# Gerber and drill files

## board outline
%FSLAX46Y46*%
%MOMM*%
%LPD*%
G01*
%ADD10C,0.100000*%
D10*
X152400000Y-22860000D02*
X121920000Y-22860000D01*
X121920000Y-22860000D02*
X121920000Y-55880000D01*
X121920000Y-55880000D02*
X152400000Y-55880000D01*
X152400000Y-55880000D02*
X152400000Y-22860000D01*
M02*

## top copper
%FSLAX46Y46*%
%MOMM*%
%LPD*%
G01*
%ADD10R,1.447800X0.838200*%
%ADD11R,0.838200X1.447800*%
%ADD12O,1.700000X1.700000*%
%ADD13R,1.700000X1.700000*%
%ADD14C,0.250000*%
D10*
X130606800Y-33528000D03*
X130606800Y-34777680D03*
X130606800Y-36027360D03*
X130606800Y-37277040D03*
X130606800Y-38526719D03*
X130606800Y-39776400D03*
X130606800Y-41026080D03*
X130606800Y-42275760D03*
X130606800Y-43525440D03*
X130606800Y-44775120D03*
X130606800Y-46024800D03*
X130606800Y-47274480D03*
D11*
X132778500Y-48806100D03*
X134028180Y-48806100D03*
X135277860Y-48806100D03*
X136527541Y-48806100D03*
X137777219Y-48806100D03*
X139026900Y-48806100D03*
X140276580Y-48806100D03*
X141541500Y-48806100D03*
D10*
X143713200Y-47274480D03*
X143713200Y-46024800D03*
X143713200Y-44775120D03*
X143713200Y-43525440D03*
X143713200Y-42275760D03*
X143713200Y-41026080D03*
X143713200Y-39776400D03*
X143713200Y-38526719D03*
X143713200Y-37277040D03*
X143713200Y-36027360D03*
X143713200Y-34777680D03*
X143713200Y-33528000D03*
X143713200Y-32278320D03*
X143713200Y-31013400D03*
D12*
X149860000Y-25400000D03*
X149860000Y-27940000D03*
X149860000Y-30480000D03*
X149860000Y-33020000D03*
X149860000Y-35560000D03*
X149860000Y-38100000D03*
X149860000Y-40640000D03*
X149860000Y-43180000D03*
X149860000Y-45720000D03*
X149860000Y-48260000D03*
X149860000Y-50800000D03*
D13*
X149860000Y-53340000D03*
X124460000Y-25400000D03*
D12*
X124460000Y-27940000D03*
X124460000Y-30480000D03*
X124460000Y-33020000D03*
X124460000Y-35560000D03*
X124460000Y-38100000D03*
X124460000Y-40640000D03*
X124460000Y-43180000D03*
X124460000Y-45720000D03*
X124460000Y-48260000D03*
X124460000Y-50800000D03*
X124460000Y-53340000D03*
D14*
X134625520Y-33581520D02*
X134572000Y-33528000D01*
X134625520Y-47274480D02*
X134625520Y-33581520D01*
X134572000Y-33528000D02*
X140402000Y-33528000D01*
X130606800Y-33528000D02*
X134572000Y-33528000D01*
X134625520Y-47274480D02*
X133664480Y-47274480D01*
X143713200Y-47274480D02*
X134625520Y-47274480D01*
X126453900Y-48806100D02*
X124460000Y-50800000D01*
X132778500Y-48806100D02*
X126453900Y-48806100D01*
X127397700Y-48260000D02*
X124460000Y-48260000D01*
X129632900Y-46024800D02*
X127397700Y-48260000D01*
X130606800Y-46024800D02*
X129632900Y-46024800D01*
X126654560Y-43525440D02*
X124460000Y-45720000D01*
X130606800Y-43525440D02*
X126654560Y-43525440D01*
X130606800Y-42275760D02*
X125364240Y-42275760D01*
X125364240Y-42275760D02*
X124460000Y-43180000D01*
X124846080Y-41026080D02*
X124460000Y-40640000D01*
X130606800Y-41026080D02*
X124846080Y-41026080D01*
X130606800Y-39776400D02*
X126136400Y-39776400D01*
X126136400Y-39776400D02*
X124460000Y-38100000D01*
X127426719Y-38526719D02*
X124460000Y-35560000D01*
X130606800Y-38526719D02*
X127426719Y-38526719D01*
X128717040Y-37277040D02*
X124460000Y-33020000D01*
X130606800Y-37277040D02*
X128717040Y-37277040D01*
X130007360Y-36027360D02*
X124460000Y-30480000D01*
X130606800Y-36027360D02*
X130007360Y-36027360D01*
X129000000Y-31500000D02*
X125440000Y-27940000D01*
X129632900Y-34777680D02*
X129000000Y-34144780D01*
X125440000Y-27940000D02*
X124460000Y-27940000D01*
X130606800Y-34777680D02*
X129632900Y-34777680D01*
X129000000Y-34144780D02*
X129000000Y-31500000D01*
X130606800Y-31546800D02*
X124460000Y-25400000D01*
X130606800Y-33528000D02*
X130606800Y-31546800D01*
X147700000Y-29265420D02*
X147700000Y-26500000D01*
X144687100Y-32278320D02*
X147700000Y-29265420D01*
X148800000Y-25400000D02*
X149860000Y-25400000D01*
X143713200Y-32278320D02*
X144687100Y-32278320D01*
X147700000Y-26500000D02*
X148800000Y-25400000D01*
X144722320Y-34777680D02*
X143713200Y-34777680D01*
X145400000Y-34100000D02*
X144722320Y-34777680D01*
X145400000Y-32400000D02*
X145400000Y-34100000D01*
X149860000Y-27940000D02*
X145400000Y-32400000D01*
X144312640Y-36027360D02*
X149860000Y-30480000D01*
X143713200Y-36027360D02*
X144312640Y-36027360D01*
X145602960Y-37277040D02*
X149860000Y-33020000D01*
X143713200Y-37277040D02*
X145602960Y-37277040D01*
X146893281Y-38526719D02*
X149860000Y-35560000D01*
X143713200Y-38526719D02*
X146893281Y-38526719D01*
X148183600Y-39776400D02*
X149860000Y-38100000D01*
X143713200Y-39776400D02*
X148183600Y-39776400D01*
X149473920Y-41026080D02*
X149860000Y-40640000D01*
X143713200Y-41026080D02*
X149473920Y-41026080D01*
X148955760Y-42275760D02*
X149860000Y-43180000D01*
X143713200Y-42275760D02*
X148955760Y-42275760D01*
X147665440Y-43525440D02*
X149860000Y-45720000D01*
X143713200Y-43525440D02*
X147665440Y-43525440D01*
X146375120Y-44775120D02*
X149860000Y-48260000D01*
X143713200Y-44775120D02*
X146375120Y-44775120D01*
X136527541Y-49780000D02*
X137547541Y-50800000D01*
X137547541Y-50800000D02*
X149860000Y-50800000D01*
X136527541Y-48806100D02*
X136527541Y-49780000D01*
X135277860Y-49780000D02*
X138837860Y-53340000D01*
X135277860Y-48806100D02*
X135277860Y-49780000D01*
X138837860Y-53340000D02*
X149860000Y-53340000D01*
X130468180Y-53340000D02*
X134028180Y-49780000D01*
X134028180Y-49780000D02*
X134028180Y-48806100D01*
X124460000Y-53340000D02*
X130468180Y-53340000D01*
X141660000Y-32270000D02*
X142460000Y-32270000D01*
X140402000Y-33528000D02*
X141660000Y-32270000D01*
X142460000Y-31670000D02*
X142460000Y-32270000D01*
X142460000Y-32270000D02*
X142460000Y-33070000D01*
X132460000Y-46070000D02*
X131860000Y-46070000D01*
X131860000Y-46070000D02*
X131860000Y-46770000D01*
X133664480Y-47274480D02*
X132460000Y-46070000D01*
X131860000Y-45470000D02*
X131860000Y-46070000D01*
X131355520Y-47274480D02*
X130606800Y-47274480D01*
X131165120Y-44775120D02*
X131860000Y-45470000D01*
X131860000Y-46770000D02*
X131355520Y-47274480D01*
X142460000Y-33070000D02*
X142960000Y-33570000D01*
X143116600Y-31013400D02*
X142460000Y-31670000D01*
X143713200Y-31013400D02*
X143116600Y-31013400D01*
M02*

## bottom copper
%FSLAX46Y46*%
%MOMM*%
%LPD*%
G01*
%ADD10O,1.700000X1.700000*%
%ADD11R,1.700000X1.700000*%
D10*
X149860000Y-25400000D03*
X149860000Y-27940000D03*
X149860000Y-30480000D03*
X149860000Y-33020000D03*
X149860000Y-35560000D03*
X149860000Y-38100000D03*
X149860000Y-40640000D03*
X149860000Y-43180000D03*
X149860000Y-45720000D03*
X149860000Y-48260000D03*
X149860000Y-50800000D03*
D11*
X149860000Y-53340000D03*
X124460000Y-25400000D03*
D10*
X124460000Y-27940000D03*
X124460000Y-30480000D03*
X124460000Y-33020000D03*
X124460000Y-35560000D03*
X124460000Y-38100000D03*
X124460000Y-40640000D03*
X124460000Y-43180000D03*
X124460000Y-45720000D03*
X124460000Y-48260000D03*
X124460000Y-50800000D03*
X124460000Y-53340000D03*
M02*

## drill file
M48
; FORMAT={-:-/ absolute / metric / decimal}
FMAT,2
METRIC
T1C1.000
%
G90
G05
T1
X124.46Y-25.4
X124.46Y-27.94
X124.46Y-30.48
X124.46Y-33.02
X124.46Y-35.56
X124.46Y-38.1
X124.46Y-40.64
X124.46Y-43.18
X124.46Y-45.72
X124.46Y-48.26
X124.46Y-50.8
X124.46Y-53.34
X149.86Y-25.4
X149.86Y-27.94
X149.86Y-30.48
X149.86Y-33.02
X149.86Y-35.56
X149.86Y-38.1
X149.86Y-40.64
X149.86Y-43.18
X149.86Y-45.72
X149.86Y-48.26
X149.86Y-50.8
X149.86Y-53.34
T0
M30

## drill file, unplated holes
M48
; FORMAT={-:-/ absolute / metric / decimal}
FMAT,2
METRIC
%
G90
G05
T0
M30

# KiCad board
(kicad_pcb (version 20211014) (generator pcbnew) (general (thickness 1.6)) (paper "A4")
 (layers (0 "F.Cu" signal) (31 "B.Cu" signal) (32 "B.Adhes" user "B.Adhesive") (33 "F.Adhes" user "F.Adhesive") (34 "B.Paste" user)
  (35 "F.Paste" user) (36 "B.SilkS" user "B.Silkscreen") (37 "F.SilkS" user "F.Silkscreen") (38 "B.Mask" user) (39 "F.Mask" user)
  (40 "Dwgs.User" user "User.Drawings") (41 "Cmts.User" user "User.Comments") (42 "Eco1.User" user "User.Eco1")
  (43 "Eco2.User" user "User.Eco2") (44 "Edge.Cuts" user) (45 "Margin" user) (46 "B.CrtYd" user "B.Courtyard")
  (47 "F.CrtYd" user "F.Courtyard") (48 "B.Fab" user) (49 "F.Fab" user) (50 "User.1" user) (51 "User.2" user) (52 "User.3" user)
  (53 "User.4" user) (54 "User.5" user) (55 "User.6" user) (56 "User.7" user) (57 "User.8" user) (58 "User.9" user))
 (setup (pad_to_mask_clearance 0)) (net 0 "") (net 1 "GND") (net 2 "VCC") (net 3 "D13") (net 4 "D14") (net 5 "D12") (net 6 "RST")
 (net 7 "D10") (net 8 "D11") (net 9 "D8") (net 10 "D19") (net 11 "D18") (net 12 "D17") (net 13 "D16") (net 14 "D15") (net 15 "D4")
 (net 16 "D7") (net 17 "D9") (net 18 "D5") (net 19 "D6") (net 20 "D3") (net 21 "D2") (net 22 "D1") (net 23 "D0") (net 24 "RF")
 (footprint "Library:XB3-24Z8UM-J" (layer "F.Cu") (at 137.16 39.37)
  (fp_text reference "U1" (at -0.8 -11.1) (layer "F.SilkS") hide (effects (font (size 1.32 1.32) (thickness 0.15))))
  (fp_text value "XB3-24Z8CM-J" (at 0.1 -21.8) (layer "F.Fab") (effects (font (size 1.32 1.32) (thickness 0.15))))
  (pad "1" smd rect (at -6.5532 -5.842) (size 1.4478 0.8382) (layers "F.Cu" "F.Paste" "F.Mask") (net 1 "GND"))
  (pad "2" smd rect (at -6.5532 -4.59232) (size 1.4478 0.8382) (layers "F.Cu" "F.Paste" "F.Mask") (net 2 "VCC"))
  (pad "3" smd rect (at -6.5532 -3.34264) (size 1.4478 0.8382) (layers "F.Cu" "F.Paste" "F.Mask") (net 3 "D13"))
  (pad "4" smd rect (at -6.5532 -2.09296) (size 1.4478 0.8382) (layers "F.Cu" "F.Paste" "F.Mask") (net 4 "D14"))
  (pad "5" smd rect (at -6.5532 -0.843281) (size 1.4478 0.8382) (layers "F.Cu" "F.Paste" "F.Mask") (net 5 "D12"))
  (pad "6" smd rect (at -6.5532 0.4064) (size 1.4478 0.8382) (layers "F.Cu" "F.Paste" "F.Mask") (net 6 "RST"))
  (pad "7" smd rect (at -6.5532 1.65608) (size 1.4478 0.8382) (layers "F.Cu" "F.Paste" "F.Mask") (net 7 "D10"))
  (pad "8" smd rect (at -6.5532 2.90576) (size 1.4478 0.8382) (layers "F.Cu" "F.Paste" "F.Mask") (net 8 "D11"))
  (pad "9" smd rect (at -6.5532 4.15544) (size 1.4478 0.8382) (layers "F.Cu" "F.Paste" "F.Mask") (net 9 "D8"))
  (pad "10" smd rect (at -6.5532 5.40512) (size 1.4478 0.8382) (layers "F.Cu" "F.Paste" "F.Mask") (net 1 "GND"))
  (pad "11" smd rect (at -6.5532 6.6548) (size 1.4478 0.8382) (layers "F.Cu" "F.Paste" "F.Mask") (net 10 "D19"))
  (pad "12" smd rect (at -6.5532 7.90448) (size 1.4478 0.8382) (layers "F.Cu" "F.Paste" "F.Mask") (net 1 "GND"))
  (pad "13" smd rect (at -4.3815 9.4361 90) (size 1.4478 0.8382) (layers "F.Cu" "F.Paste" "F.Mask") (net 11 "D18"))
  (pad "14" smd rect (at -3.13182 9.4361 90) (size 1.4478 0.8382) (layers "F.Cu" "F.Paste" "F.Mask") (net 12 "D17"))
  (pad "15" smd rect (at -1.88214 9.4361 90) (size 1.4478 0.8382) (layers "F.Cu" "F.Paste" "F.Mask") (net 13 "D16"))
  (pad "16" smd rect (at -0.632459 9.4361 90) (size 1.4478 0.8382) (layers "F.Cu" "F.Paste" "F.Mask") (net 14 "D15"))
  (pad "17" smd rect (at 0.617219 9.4361 90) (size 1.4478 0.8382) (layers "F.Cu" "F.Paste" "F.Mask"))
  (pad "18" smd rect (at 1.8669 9.4361 90) (size 1.4478 0.8382) (layers "F.Cu" "F.Paste" "F.Mask"))
  (pad "19" smd rect (at 3.11658 9.4361 90) (size 1.4478 0.8382) (layers "F.Cu" "F.Paste" "F.Mask"))
  (pad "20" smd rect (at 4.3815 9.4361 90) (size 1.4478 0.8382) (layers "F.Cu" "F.Paste" "F.Mask"))
  (pad "21" smd rect (at 6.5532 7.90448) (size 1.4478 0.8382) (layers "F.Cu" "F.Paste" "F.Mask") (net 1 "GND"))
  (pad "22" smd rect (at 6.5532 6.6548) (size 1.4478 0.8382) (layers "F.Cu" "F.Paste" "F.Mask"))
  (pad "23" smd rect (at 6.5532 5.40512) (size 1.4478 0.8382) (layers "F.Cu" "F.Paste" "F.Mask") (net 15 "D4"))
  (pad "24" smd rect (at 6.5532 4.15544) (size 1.4478 0.8382) (layers "F.Cu" "F.Paste" "F.Mask") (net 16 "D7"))
  (pad "25" smd rect (at 6.5532 2.90576) (size 1.4478 0.8382) (layers "F.Cu" "F.Paste" "F.Mask") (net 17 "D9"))
  (pad "26" smd rect (at 6.5532 1.65608) (size 1.4478 0.8382) (layers "F.Cu" "F.Paste" "F.Mask") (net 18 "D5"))
  (pad "27" smd rect (at 6.5532 0.4064) (size 1.4478 0.8382) (layers "F.Cu" "F.Paste" "F.Mask") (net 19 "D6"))
  (pad "28" smd rect (at 6.5532 -0.843281) (size 1.4478 0.8382) (layers "F.Cu" "F.Paste" "F.Mask") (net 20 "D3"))
  (pad "29" smd rect (at 6.5532 -2.09296) (size 1.4478 0.8382) (layers "F.Cu" "F.Paste" "F.Mask") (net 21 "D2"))
  (pad "30" smd rect (at 6.5532 -3.34264) (size 1.4478 0.8382) (layers "F.Cu" "F.Paste" "F.Mask") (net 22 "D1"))
  (pad "31" smd rect (at 6.5532 -4.59232) (size 1.4478 0.8382) (layers "F.Cu" "F.Paste" "F.Mask") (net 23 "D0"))
  (pad "32" smd rect (at 6.5532 -5.842) (size 1.4478 0.8382) (layers "F.Cu" "F.Paste" "F.Mask") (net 1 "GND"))
  (pad "33" smd rect (at 6.5532 -7.09168) (size 1.4478 0.8382) (layers "F.Cu" "F.Paste" "F.Mask") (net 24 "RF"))
  (pad "34" smd rect (at 6.5532 -8.3566) (size 1.4478 0.8382) (layers "F.Cu" "F.Paste" "F.Mask") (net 1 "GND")))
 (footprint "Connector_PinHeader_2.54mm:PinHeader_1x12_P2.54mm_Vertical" (layer "F.Cu") (at 124.46 25.4)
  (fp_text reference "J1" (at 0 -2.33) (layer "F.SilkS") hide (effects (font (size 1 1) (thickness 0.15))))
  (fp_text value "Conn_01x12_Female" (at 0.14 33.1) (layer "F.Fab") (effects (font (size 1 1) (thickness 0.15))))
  (pad "1" thru_hole rect (at 0 0) (size 1.7 1.7) (drill 1) (layers *.Cu *.Mask) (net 1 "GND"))
  (pad "2" thru_hole oval (at 0 2.54) (size 1.7 1.7) (drill 1) (layers *.Cu *.Mask) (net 2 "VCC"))
  (pad "3" thru_hole oval (at 0 5.08) (size 1.7 1.7) (drill 1) (layers *.Cu *.Mask) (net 3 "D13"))
  (pad "4" thru_hole oval (at 0 7.62) (size 1.7 1.7) (drill 1) (layers *.Cu *.Mask) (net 4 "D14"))
  (pad "5" thru_hole oval (at 0 10.16) (size 1.7 1.7) (drill 1) (layers *.Cu *.Mask) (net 5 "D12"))
  (pad "6" thru_hole oval (at 0 12.7) (size 1.7 1.7) (drill 1) (layers *.Cu *.Mask) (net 6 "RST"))
  (pad "7" thru_hole oval (at 0 15.24) (size 1.7 1.7) (drill 1) (layers *.Cu *.Mask) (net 7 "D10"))
  (pad "8" thru_hole oval (at 0 17.78) (size 1.7 1.7) (drill 1) (layers *.Cu *.Mask) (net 8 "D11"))
  (pad "9" thru_hole oval (at 0 20.32) (size 1.7 1.7) (drill 1) (layers *.Cu *.Mask) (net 9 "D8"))
  (pad "10" thru_hole oval (at 0 22.86) (size 1.7 1.7) (drill 1) (layers *.Cu *.Mask) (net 10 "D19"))
  (pad "11" thru_hole oval (at 0 25.4) (size 1.7 1.7) (drill 1) (layers *.Cu *.Mask) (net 11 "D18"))
  (pad "12" thru_hole oval (at 0 27.94) (size 1.7 1.7) (drill 1) (layers *.Cu *.Mask) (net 12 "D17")))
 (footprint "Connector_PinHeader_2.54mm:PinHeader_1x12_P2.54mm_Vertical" (layer "F.Cu") (at 149.86 53.34 180)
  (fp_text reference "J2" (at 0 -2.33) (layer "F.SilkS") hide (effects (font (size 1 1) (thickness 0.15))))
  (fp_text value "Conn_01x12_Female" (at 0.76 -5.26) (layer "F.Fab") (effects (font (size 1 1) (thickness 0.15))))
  (pad "1" thru_hole rect (at 0 0 180) (size 1.7 1.7) (drill 1) (layers *.Cu *.Mask) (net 13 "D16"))
  (pad "2" thru_hole oval (at 0 2.54 180) (size 1.7 1.7) (drill 1) (layers *.Cu *.Mask) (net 14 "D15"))
  (pad "3" thru_hole oval (at 0 5.08 180) (size 1.7 1.7) (drill 1) (layers *.Cu *.Mask) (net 15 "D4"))
  (pad "4" thru_hole oval (at 0 7.62 180) (size 1.7 1.7) (drill 1) (layers *.Cu *.Mask) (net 16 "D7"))
  (pad "5" thru_hole oval (at 0 10.16 180) (size 1.7 1.7) (drill 1) (layers *.Cu *.Mask) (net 17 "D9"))
  (pad "6" thru_hole oval (at 0 12.7 180) (size 1.7 1.7) (drill 1) (layers *.Cu *.Mask) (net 18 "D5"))
  (pad "7" thru_hole oval (at 0 15.24 180) (size 1.7 1.7) (drill 1) (layers *.Cu *.Mask) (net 19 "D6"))
  (pad "8" thru_hole oval (at 0 17.78 180) (size 1.7 1.7) (drill 1) (layers *.Cu *.Mask) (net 20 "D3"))
  (pad "9" thru_hole oval (at 0 20.32 180) (size 1.7 1.7) (drill 1) (layers *.Cu *.Mask) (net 21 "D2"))
  (pad "10" thru_hole oval (at 0 22.86 180) (size 1.7 1.7) (drill 1) (layers *.Cu *.Mask) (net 22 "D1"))
  (pad "11" thru_hole oval (at 0 25.4 180) (size 1.7 1.7) (drill 1) (layers *.Cu *.Mask) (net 23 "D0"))
  (pad "12" thru_hole oval (at 0 27.94 180) (size 1.7 1.7) (drill 1) (layers *.Cu *.Mask) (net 24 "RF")))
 (gr_rect (start 152.4 22.86) (end 121.92 55.88) (layer "Edge.Cuts") (width 0.1) (fill none))
 (segment (start 130.6068 39.7764) (end 126.1364 39.7764) (width 0.25) (layer "F.Cu") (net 6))
 (segment (start 126.1364 39.7764) (end 124.46 38.1) (width 0.25) (layer "F.Cu") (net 6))
 (segment (start 145.4 34.1) (end 144.72232 34.77768) (width 0.25) (layer "F.Cu") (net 23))
 (segment (start 149.86 27.94) (end 145.4 32.4) (width 0.25) (layer "F.Cu") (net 23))
 (segment (start 145.4 32.4) (end 145.4 34.1) (width 0.25) (layer "F.Cu") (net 23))
 (segment (start 144.72232 34.77768) (end 143.7132 34.77768) (width 0.25) (layer "F.Cu") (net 23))
 (segment (start 144.31264 36.02736) (end 149.86 30.48) (width 0.25) (layer "F.Cu") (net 22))
 (segment (start 143.7132 36.02736) (end 144.31264 36.02736) (width 0.25) (layer "F.Cu") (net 22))
 (segment (start 143.7132 37.27704) (end 145.60296 37.27704) (width 0.25) (layer "F.Cu") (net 21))
 (segment (start 145.60296 37.27704) (end 149.86 33.02) (width 0.25) (layer "F.Cu") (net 21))
 (segment (start 146.893281 38.526719) (end 149.86 35.56) (width 0.25) (layer "F.Cu") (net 20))
 (segment (start 143.7132 38.526719) (end 146.893281 38.526719) (width 0.25) (layer "F.Cu") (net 20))
 (segment (start 143.7132 44.77512) (end 146.37512 44.77512) (width 0.25) (layer "F.Cu") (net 15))
 (segment (start 146.37512 44.77512) (end 149.86 48.26) (width 0.25) (layer "F.Cu") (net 15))
 (segment (start 149.47392 41.02608) (end 149.86 40.64) (width 0.25) (layer "F.Cu") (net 18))
 (segment (start 143.7132 41.02608) (end 149.47392 41.02608) (width 0.25) (layer "F.Cu") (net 18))
 (segment (start 148.1836 39.7764) (end 149.86 38.1) (width 0.25) (layer "F.Cu") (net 19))
 (segment (start 143.7132 39.7764) (end 148.1836 39.7764) (width 0.25) (layer "F.Cu") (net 19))
 (segment (start 147.66544 43.52544) (end 149.86 45.72) (width 0.25) (layer "F.Cu") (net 16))
 (segment (start 143.7132 43.52544) (end 147.66544 43.52544) (width 0.25) (layer "F.Cu") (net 16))
 (segment (start 126.65456 43.52544) (end 124.46 45.72) (width 0.25) (layer "F.Cu") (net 9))
 (segment (start 130.6068 43.52544) (end 126.65456 43.52544) (width 0.25) (layer "F.Cu") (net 9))
 (segment (start 148.95576 42.27576) (end 149.86 43.18) (width 0.25) (layer "F.Cu") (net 17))
 (segment (start 143.7132 42.27576) (end 148.95576 42.27576) (width 0.25) (layer "F.Cu") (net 17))
 (segment (start 130.6068 41.02608) (end 124.84608 41.02608) (width 0.25) (layer "F.Cu") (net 7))
 (segment (start 124.84608 41.02608) (end 124.46 40.64) (width 0.25) (layer "F.Cu") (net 7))
 (segment (start 130.6068 46.0248) (end 129.6329 46.0248) (width 0.25) (layer "F.Cu") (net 10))
 (segment (start 127.3977 48.26) (end 124.46 48.26) (width 0.25) (layer "F.Cu") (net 10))
 (segment (start 129.6329 46.0248) (end 127.3977 48.26) (width 0.25) (layer "F.Cu") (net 10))
 (segment (start 132.7785 48.8061) (end 126.4539 48.8061) (width 0.25) (layer "F.Cu") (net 11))
 (segment (start 126.4539 48.8061) (end 124.46 50.8) (width 0.25) (layer "F.Cu") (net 11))
 (segment (start 124.46 53.34) (end 130.46818 53.34) (width 0.25) (layer "F.Cu") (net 12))
 (segment (start 134.02818 49.78) (end 134.02818 48.8061) (width 0.25) (layer "F.Cu") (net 12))
 (segment (start 130.46818 53.34) (end 134.02818 49.78) (width 0.25) (layer "F.Cu") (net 12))
 (segment (start 135.27786 49.78) (end 138.83786 53.34) (width 0.25) (layer "F.Cu") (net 13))
 (segment (start 138.83786 53.34) (end 149.86 53.34) (width 0.25) (layer "F.Cu") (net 13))
 (segment (start 135.27786 48.8061) (end 135.27786 49.78) (width 0.25) (layer "F.Cu") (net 13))
 (segment (start 137.547541 50.8) (end 149.86 50.8) (width 0.25) (layer "F.Cu") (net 14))
 (segment (start 136.527541 49.78) (end 137.547541 50.8) (width 0.25) (layer "F.Cu") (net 14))
 (segment (start 136.527541 48.8061) (end 136.527541 49.78) (width 0.25) (layer "F.Cu") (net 14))
 (segment (start 130.6068 37.27704) (end 128.71704 37.27704) (width 0.25) (layer "F.Cu") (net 4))
 (segment (start 128.71704 37.27704) (end 124.46 33.02) (width 0.25) (layer "F.Cu") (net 4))
 (segment (start 130.00736 36.02736) (end 124.46 30.48) (width 0.25) (layer "F.Cu") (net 3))
 (segment (start 130.6068 36.02736) (end 130.00736 36.02736) (width 0.25) (layer "F.Cu") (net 3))
 (segment (start 127.426719 38.526719) (end 124.46 35.56) (width 0.25) (layer "F.Cu") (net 5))
 (segment (start 130.6068 38.526719) (end 127.426719 38.526719) (width 0.25) (layer "F.Cu") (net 5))
 (segment (start 130.6068 42.27576) (end 125.36424 42.27576) (width 0.25) (layer "F.Cu") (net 8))
 (segment (start 125.36424 42.27576) (end 124.46 43.18) (width 0.25) (layer "F.Cu") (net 8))
 (segment (start 143.7132 32.27832) (end 144.6871 32.27832) (width 0.25) (layer "F.Cu") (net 24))
 (segment (start 144.6871 32.27832) (end 147.7 29.26542) (width 0.25) (layer "F.Cu") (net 24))
 (segment (start 148.8 25.4) (end 149.86 25.4) (width 0.25) (layer "F.Cu") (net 24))
 (segment (start 147.7 26.5) (end 148.8 25.4) (width 0.25) (layer "F.Cu") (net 24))
 (segment (start 147.7 29.26542) (end 147.7 26.5) (width 0.25) (layer "F.Cu") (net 24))
 (segment (start 130.6068 33.528) (end 134.572 33.528) (width 0.25) (layer "F.Cu") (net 1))
 (segment (start 142.46 31.67) (end 142.46 32.27) (width 0.25) (layer "F.Cu") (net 1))
 (segment (start 131.86 46.77) (end 131.35552 47.27448) (width 0.25) (layer "F.Cu") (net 1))
 (segment (start 143.7132 31.0134) (end 143.1166 31.0134) (width 0.25) (layer "F.Cu") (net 1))
 (segment (start 131.35552 47.27448) (end 130.6068 47.27448) (width 0.25) (layer "F.Cu") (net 1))
 (segment (start 134.62552 47.27448) (end 134.62552 33.58152) (width 0.25) (layer "F.Cu") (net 1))
 (segment (start 134.572 33.528) (end 140.402 33.528) (width 0.25) (layer "F.Cu") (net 1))
 (segment (start 131.16512 44.77512) (end 131.86 45.47) (width 0.25) (layer "F.Cu") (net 1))
 (segment (start 142.46 32.27) (end 142.46 33.07) (width 0.25) (layer "F.Cu") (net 1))
 (segment (start 142.46 33.07) (end 142.96 33.57) (width 0.25) (layer "F.Cu") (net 1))
 (segment (start 140.402 33.528) (end 141.66 32.27) (width 0.25) (layer "F.Cu") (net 1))
 (segment (start 134.62552 33.58152) (end 134.572 33.528) (width 0.25) (layer "F.Cu") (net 1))
 (segment (start 133.66448 47.27448) (end 132.46 46.07) (width 0.25) (layer "F.Cu") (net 1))
 (segment (start 130.6068 31.5468) (end 124.46 25.4) (width 0.25) (layer "F.Cu") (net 1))
 (segment (start 143.1166 31.0134) (end 142.46 31.67) (width 0.25) (layer "F.Cu") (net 1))
 (segment (start 134.62552 47.27448) (end 133.66448 47.27448) (width 0.25) (layer "F.Cu") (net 1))
 (segment (start 131.86 45.47) (end 131.86 46.07) (width 0.25) (layer "F.Cu") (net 1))
 (segment (start 141.66 32.27) (end 142.46 32.27) (width 0.25) (layer "F.Cu") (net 1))
 (segment (start 143.7132 47.27448) (end 134.62552 47.27448) (width 0.25) (layer "F.Cu") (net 1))
 (segment (start 130.6068 33.528) (end 130.6068 31.5468) (width 0.25) (layer "F.Cu") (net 1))
 (segment (start 132.46 46.07) (end 131.86 46.07) (width 0.25) (layer "F.Cu") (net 1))
 (segment (start 131.86 46.07) (end 131.86 46.77) (width 0.25) (layer "F.Cu") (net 1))
 (segment (start 130.6068 34.77768) (end 129.6329 34.77768) (width 0.25) (layer "F.Cu") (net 2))
 (segment (start 129.6329 34.77768) (end 129 34.14478) (width 0.25) (layer "F.Cu") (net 2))
 (segment (start 129 31.5) (end 125.44 27.94) (width 0.25) (layer "F.Cu") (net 2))
 (segment (start 125.44 27.94) (end 124.46 27.94) (width 0.25) (layer "F.Cu") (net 2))
 (segment (start 129 34.14478) (end 129 31.5) (width 0.25) (layer "F.Cu") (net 2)))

